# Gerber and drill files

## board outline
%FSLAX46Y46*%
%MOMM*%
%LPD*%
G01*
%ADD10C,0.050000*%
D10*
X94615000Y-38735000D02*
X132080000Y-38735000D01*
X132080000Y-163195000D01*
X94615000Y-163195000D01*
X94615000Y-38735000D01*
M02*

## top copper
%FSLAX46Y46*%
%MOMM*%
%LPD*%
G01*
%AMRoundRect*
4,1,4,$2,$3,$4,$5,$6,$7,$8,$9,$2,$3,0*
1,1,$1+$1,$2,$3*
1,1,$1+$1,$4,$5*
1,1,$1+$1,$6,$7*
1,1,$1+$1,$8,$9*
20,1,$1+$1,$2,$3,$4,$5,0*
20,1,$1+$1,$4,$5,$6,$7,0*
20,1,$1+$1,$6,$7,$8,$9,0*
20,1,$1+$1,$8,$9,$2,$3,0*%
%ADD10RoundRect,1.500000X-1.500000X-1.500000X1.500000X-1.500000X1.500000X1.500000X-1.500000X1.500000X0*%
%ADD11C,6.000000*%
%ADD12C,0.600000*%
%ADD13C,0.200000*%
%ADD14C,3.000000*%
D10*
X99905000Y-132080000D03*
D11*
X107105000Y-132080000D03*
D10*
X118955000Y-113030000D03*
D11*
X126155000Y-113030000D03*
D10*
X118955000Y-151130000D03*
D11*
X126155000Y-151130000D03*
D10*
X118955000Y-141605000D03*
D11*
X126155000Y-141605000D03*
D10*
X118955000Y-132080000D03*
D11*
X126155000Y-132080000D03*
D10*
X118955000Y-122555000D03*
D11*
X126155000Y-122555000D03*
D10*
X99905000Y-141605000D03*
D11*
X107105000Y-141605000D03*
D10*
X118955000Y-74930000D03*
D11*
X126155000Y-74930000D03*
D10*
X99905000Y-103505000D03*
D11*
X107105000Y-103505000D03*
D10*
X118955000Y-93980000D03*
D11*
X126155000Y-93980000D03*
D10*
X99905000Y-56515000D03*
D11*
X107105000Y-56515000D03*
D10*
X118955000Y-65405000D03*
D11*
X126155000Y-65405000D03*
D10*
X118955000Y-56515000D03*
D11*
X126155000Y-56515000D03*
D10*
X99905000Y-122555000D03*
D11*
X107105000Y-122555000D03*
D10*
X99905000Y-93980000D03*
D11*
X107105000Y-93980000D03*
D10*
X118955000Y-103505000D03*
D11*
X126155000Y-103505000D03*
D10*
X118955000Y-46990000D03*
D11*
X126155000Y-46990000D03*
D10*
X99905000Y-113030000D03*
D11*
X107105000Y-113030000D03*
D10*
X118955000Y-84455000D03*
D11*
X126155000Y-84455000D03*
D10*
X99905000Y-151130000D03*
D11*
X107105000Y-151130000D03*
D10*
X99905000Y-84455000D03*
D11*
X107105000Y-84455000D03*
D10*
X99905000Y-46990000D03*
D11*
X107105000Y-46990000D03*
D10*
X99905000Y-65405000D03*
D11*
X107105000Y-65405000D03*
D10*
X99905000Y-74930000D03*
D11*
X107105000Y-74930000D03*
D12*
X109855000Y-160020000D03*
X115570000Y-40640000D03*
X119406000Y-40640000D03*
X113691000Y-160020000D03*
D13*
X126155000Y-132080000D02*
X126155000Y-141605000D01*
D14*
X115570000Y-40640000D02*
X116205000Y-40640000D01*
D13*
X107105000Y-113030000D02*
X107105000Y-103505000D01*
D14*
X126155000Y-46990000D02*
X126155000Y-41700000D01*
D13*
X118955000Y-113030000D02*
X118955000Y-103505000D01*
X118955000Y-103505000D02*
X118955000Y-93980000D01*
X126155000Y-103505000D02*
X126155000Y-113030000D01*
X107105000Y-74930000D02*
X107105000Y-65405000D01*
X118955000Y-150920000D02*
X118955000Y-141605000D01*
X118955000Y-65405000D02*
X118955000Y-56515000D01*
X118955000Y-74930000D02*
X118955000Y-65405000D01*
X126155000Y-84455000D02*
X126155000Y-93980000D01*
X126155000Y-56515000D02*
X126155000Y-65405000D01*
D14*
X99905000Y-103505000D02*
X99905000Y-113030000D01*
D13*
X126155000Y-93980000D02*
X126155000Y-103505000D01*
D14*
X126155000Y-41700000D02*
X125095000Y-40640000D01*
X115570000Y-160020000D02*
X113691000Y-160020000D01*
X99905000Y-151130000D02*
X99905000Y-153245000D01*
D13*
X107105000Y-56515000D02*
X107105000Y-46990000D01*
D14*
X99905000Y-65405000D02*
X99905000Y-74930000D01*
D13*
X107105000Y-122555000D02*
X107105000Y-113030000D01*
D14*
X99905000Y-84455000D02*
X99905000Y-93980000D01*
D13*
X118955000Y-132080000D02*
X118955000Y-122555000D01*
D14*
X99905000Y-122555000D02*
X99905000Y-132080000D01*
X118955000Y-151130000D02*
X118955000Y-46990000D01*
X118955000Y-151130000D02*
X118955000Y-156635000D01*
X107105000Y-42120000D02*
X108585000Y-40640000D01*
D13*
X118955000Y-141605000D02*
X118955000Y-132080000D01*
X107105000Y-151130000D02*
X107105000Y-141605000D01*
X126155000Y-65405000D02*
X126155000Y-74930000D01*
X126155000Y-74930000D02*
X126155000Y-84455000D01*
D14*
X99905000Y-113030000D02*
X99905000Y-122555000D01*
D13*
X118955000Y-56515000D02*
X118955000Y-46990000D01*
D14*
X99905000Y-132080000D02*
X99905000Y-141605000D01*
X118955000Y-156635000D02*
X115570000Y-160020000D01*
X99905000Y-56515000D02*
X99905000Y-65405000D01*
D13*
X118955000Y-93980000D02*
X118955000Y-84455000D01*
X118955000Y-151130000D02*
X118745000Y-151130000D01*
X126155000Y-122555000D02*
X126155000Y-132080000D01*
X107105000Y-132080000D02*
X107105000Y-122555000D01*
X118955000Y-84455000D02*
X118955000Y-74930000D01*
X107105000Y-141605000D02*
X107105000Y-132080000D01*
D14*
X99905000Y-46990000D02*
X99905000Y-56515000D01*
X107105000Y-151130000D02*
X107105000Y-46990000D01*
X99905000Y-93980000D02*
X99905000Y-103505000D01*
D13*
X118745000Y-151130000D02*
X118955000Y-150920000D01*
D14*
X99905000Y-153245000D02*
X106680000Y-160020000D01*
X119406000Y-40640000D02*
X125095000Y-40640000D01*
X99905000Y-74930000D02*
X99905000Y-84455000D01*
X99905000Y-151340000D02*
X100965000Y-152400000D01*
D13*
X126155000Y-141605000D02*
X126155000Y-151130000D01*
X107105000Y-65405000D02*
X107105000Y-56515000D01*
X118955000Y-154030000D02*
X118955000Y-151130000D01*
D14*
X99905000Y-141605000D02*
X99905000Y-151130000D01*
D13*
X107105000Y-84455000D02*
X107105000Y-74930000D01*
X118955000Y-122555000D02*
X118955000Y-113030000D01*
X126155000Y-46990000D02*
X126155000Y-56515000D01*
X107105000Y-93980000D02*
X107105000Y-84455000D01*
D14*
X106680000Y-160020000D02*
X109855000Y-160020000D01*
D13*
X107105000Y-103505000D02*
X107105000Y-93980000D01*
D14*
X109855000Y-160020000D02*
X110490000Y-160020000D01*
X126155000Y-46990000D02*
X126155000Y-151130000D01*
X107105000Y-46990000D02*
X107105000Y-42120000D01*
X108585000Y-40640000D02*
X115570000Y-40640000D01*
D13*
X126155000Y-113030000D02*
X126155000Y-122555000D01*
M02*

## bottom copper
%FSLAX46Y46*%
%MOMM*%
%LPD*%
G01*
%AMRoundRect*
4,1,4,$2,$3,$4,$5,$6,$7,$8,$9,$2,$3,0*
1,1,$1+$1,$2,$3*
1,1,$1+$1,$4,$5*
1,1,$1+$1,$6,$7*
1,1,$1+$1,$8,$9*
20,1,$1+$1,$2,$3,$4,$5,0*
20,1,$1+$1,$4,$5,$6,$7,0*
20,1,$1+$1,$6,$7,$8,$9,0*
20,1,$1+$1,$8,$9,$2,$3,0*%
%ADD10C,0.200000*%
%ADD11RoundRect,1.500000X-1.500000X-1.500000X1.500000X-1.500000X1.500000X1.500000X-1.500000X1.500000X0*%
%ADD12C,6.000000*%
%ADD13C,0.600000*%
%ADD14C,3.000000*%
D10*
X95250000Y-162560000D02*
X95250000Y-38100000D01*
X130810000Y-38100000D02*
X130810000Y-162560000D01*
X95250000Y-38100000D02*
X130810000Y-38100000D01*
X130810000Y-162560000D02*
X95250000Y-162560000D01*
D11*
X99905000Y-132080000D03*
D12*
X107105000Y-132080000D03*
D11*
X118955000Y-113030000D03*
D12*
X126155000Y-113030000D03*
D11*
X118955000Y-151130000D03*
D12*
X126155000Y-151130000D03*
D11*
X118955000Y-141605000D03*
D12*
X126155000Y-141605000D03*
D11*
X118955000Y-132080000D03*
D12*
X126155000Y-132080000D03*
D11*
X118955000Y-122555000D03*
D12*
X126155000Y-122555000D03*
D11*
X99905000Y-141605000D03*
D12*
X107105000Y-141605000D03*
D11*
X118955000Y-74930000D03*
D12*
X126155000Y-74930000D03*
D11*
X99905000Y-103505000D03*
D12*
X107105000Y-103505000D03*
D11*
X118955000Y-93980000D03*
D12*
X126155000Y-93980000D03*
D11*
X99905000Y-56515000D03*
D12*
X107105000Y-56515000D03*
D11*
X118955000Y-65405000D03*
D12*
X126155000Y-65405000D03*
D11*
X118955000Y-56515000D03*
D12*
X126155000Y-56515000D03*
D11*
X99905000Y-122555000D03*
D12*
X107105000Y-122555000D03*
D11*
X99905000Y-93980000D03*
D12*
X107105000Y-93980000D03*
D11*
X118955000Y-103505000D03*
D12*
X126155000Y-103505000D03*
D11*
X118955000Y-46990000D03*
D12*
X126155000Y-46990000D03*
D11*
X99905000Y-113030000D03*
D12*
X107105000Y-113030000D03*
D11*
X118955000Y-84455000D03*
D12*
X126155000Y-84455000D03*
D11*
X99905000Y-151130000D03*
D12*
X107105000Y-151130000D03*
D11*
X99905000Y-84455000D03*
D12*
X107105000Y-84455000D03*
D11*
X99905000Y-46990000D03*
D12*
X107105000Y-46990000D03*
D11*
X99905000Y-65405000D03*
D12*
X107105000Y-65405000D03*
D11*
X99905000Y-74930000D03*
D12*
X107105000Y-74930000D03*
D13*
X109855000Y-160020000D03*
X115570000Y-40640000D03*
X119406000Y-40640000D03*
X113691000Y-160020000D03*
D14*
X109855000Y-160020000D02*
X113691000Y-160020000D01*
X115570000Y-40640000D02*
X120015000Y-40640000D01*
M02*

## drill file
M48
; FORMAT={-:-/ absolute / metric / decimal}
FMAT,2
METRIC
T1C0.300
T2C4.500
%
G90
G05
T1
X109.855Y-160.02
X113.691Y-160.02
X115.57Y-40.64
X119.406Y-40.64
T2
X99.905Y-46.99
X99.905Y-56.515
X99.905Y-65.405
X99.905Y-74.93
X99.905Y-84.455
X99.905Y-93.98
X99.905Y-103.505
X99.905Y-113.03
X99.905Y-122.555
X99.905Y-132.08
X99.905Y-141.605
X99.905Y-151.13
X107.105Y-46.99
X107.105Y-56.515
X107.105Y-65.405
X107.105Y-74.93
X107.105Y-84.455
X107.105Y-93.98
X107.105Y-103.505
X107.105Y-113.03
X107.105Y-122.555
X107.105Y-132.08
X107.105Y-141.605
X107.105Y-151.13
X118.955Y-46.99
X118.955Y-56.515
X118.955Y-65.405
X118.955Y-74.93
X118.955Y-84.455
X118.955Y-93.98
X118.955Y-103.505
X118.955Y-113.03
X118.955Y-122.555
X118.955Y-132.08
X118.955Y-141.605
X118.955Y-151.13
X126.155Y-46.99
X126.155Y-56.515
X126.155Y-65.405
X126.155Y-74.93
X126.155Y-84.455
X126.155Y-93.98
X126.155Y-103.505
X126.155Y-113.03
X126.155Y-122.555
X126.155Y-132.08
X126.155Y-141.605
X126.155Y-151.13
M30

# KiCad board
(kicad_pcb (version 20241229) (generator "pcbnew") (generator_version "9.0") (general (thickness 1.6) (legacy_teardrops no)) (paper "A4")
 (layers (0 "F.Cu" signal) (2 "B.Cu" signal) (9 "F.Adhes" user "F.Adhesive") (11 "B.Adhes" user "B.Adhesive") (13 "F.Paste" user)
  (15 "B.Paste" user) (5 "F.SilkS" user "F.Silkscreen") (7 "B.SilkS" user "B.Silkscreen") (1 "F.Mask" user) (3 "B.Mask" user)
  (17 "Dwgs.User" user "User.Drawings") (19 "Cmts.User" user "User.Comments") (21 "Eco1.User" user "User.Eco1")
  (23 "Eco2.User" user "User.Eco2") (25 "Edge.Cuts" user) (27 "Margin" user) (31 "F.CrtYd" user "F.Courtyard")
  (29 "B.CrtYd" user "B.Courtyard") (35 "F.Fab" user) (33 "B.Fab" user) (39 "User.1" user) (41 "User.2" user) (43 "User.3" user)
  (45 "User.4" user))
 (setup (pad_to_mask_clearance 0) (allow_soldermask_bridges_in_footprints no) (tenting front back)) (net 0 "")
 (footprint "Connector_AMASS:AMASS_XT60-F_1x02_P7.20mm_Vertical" (layer "F.Cu") (at 99.905 132.08)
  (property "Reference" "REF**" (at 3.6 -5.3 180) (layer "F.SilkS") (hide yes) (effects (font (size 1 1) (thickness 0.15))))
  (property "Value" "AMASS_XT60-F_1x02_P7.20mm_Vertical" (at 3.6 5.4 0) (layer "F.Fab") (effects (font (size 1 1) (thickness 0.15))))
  (pad "1" thru_hole roundrect (at 0 0) (size 6 6) (drill 4.5) (layers "*.Cu" "*.Mask") (remove_unused_layers no) (roundrect_rratio 0.25))
  (pad "2" thru_hole circle (at 7.2 0) (size 6 6) (drill 4.5) (layers "*.Cu" "*.Mask") (remove_unused_layers no)))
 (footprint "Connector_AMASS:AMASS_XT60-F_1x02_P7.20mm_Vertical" (layer "F.Cu") (at 118.955 113.03)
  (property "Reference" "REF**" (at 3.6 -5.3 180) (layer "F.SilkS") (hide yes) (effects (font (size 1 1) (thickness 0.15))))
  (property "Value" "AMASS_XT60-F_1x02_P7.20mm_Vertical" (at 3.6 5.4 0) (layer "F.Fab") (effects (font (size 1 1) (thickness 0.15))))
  (pad "1" thru_hole roundrect (at 0 0) (size 6 6) (drill 4.5) (layers "*.Cu" "*.Mask") (remove_unused_layers no) (roundrect_rratio 0.25))
  (pad "2" thru_hole circle (at 7.2 0) (size 6 6) (drill 4.5) (layers "*.Cu" "*.Mask") (remove_unused_layers no)))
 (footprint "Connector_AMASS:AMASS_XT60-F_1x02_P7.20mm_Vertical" (layer "F.Cu") (at 118.955 151.13)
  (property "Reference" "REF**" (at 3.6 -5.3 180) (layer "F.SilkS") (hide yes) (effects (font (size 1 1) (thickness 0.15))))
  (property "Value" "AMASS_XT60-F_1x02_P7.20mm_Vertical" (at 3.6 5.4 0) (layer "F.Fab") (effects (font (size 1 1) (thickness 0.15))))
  (pad "1" thru_hole roundrect (at 0 0) (size 6 6) (drill 4.5) (layers "*.Cu" "*.Mask") (remove_unused_layers no) (roundrect_rratio 0.25))
  (pad "2" thru_hole circle (at 7.2 0) (size 6 6) (drill 4.5) (layers "*.Cu" "*.Mask") (remove_unused_layers no)))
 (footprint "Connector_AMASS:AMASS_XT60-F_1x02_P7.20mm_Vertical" (layer "F.Cu") (at 118.955 141.605)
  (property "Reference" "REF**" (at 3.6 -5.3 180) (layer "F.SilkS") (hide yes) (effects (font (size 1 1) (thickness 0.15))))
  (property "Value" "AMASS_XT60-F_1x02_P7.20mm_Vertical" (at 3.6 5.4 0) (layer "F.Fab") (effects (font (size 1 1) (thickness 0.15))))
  (pad "1" thru_hole roundrect (at 0 0) (size 6 6) (drill 4.5) (layers "*.Cu" "*.Mask") (remove_unused_layers no) (roundrect_rratio 0.25))
  (pad "2" thru_hole circle (at 7.2 0) (size 6 6) (drill 4.5) (layers "*.Cu" "*.Mask") (remove_unused_layers no)))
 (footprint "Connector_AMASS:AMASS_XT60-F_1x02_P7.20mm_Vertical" (layer "F.Cu") (at 118.955 132.08)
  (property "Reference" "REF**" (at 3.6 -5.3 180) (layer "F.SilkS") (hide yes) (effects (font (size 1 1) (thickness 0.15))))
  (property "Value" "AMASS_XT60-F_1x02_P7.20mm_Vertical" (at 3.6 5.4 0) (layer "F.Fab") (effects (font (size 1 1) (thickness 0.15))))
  (pad "1" thru_hole roundrect (at 0 0) (size 6 6) (drill 4.5) (layers "*.Cu" "*.Mask") (remove_unused_layers no) (roundrect_rratio 0.25))
  (pad "2" thru_hole circle (at 7.2 0) (size 6 6) (drill 4.5) (layers "*.Cu" "*.Mask") (remove_unused_layers no)))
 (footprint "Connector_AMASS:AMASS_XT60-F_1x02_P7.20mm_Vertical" (layer "F.Cu") (at 118.955 122.555)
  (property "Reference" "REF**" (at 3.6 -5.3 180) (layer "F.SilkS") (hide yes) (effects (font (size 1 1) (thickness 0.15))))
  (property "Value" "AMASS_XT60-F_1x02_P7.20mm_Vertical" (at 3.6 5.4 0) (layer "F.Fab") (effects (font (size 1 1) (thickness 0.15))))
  (pad "1" thru_hole roundrect (at 0 0) (size 6 6) (drill 4.5) (layers "*.Cu" "*.Mask") (remove_unused_layers no) (roundrect_rratio 0.25))
  (pad "2" thru_hole circle (at 7.2 0) (size 6 6) (drill 4.5) (layers "*.Cu" "*.Mask") (remove_unused_layers no)))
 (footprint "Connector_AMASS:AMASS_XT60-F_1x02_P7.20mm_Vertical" (layer "F.Cu") (at 99.905 141.605)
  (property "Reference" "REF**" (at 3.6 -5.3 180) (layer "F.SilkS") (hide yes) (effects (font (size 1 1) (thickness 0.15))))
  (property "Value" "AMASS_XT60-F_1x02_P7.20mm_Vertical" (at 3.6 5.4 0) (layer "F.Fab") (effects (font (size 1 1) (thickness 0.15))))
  (pad "1" thru_hole roundrect (at 0 0) (size 6 6) (drill 4.5) (layers "*.Cu" "*.Mask") (remove_unused_layers no) (roundrect_rratio 0.25))
  (pad "2" thru_hole circle (at 7.2 0) (size 6 6) (drill 4.5) (layers "*.Cu" "*.Mask") (remove_unused_layers no)))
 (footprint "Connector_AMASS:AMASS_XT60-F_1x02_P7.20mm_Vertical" (layer "F.Cu") (at 118.955 74.93)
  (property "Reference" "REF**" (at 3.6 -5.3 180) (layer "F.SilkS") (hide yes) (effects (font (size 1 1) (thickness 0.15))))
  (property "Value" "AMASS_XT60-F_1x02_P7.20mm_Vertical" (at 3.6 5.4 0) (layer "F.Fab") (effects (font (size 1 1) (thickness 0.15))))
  (pad "1" thru_hole roundrect (at 0 0) (size 6 6) (drill 4.5) (layers "*.Cu" "*.Mask") (remove_unused_layers no) (roundrect_rratio 0.25))
  (pad "2" thru_hole circle (at 7.2 0) (size 6 6) (drill 4.5) (layers "*.Cu" "*.Mask") (remove_unused_layers no)))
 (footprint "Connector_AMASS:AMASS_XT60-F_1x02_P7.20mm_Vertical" (layer "F.Cu") (at 99.905 103.505)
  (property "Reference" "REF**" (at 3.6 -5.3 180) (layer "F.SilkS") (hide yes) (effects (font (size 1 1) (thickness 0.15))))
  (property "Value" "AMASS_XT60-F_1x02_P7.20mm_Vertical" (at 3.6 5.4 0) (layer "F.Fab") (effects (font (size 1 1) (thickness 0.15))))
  (pad "1" thru_hole roundrect (at 0 0) (size 6 6) (drill 4.5) (layers "*.Cu" "*.Mask") (remove_unused_layers no) (roundrect_rratio 0.25))
  (pad "2" thru_hole circle (at 7.2 0) (size 6 6) (drill 4.5) (layers "*.Cu" "*.Mask") (remove_unused_layers no)))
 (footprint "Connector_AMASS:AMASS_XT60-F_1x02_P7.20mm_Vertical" (layer "F.Cu") (at 118.955 93.98)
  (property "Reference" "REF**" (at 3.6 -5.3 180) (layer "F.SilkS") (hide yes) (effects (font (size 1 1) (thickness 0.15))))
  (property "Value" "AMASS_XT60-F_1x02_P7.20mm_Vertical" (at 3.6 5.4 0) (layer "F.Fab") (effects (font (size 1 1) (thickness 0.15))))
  (pad "1" thru_hole roundrect (at 0 0) (size 6 6) (drill 4.5) (layers "*.Cu" "*.Mask") (remove_unused_layers no) (roundrect_rratio 0.25))
  (pad "2" thru_hole circle (at 7.2 0) (size 6 6) (drill 4.5) (layers "*.Cu" "*.Mask") (remove_unused_layers no)))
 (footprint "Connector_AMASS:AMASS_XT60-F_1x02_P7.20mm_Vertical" (layer "F.Cu") (at 99.905 56.515)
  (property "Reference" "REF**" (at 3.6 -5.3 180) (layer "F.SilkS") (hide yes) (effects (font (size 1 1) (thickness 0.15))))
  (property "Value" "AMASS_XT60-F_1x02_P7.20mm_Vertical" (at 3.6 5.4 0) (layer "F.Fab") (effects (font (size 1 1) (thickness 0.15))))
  (pad "1" thru_hole roundrect (at 0 0) (size 6 6) (drill 4.5) (layers "*.Cu" "*.Mask") (remove_unused_layers no) (roundrect_rratio 0.25))
  (pad "2" thru_hole circle (at 7.2 0) (size 6 6) (drill 4.5) (layers "*.Cu" "*.Mask") (remove_unused_layers no)))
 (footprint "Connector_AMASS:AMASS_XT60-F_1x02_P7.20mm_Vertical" (layer "F.Cu") (at 118.955 65.405)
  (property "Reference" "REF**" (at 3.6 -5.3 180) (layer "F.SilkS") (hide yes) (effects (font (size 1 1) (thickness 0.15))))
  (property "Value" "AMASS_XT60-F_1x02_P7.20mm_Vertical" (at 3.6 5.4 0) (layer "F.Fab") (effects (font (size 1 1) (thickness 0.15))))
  (pad "1" thru_hole roundrect (at 0 0) (size 6 6) (drill 4.5) (layers "*.Cu" "*.Mask") (remove_unused_layers no) (roundrect_rratio 0.25))
  (pad "2" thru_hole circle (at 7.2 0) (size 6 6) (drill 4.5) (layers "*.Cu" "*.Mask") (remove_unused_layers no)))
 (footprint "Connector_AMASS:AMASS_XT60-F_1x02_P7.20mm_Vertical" (layer "F.Cu") (at 118.955 56.515)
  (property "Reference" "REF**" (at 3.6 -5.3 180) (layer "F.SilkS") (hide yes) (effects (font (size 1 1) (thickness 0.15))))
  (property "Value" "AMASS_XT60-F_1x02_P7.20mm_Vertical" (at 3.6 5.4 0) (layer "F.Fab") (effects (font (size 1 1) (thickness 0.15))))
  (pad "1" thru_hole roundrect (at 0 0) (size 6 6) (drill 4.5) (layers "*.Cu" "*.Mask") (remove_unused_layers no) (roundrect_rratio 0.25))
  (pad "2" thru_hole circle (at 7.2 0) (size 6 6) (drill 4.5) (layers "*.Cu" "*.Mask") (remove_unused_layers no)))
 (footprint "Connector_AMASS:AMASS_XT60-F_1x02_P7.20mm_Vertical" (layer "F.Cu") (at 99.905 122.555)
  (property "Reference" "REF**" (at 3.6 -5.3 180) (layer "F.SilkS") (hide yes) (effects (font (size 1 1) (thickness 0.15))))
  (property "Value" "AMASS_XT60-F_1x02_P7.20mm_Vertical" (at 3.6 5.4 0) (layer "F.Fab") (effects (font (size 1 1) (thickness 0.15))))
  (pad "1" thru_hole roundrect (at 0 0) (size 6 6) (drill 4.5) (layers "*.Cu" "*.Mask") (remove_unused_layers no) (roundrect_rratio 0.25))
  (pad "2" thru_hole circle (at 7.2 0) (size 6 6) (drill 4.5) (layers "*.Cu" "*.Mask") (remove_unused_layers no)))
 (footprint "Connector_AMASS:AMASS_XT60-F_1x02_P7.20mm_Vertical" (layer "F.Cu") (at 99.905 93.98)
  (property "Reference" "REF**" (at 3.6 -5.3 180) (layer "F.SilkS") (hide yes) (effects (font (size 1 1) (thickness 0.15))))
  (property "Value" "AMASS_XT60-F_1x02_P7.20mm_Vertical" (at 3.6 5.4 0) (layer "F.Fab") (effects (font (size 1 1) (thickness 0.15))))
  (pad "1" thru_hole roundrect (at 0 0) (size 6 6) (drill 4.5) (layers "*.Cu" "*.Mask") (remove_unused_layers no) (roundrect_rratio 0.25))
  (pad "2" thru_hole circle (at 7.2 0) (size 6 6) (drill 4.5) (layers "*.Cu" "*.Mask") (remove_unused_layers no)))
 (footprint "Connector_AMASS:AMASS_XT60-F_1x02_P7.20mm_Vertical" (layer "F.Cu") (at 118.955 103.505)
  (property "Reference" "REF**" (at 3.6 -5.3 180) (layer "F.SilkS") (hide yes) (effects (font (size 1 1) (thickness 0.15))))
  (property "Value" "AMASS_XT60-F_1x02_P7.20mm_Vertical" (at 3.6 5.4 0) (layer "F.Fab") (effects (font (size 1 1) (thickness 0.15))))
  (pad "1" thru_hole roundrect (at 0 0) (size 6 6) (drill 4.5) (layers "*.Cu" "*.Mask") (remove_unused_layers no) (roundrect_rratio 0.25))
  (pad "2" thru_hole circle (at 7.2 0) (size 6 6) (drill 4.5) (layers "*.Cu" "*.Mask") (remove_unused_layers no)))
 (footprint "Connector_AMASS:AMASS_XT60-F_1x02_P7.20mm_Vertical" (layer "F.Cu") (at 118.955 46.99)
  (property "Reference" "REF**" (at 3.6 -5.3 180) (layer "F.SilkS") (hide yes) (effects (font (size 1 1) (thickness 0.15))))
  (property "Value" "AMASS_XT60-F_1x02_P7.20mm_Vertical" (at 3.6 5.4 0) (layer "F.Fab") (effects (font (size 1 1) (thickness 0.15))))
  (pad "1" thru_hole roundrect (at 0 0) (size 6 6) (drill 4.5) (layers "*.Cu" "*.Mask") (remove_unused_layers no) (roundrect_rratio 0.25))
  (pad "2" thru_hole circle (at 7.2 0) (size 6 6) (drill 4.5) (layers "*.Cu" "*.Mask") (remove_unused_layers no)))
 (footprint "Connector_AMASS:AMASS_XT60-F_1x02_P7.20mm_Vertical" (layer "F.Cu") (at 99.905 113.03)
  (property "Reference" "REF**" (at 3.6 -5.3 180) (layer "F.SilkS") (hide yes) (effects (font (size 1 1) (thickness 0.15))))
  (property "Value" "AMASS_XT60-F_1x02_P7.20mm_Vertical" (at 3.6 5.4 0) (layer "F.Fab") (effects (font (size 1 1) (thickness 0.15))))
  (pad "1" thru_hole roundrect (at 0 0) (size 6 6) (drill 4.5) (layers "*.Cu" "*.Mask") (remove_unused_layers no) (roundrect_rratio 0.25))
  (pad "2" thru_hole circle (at 7.2 0) (size 6 6) (drill 4.5) (layers "*.Cu" "*.Mask") (remove_unused_layers no)))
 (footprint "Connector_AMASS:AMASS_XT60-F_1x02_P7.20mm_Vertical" (layer "F.Cu") (at 118.955 84.455)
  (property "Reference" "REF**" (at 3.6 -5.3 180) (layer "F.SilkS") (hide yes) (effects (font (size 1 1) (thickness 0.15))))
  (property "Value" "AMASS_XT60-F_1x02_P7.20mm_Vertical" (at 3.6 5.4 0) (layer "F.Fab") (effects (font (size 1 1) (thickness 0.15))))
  (pad "1" thru_hole roundrect (at 0 0) (size 6 6) (drill 4.5) (layers "*.Cu" "*.Mask") (remove_unused_layers no) (roundrect_rratio 0.25))
  (pad "2" thru_hole circle (at 7.2 0) (size 6 6) (drill 4.5) (layers "*.Cu" "*.Mask") (remove_unused_layers no)))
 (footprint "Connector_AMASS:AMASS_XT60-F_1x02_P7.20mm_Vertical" (layer "F.Cu") (at 99.905 151.13)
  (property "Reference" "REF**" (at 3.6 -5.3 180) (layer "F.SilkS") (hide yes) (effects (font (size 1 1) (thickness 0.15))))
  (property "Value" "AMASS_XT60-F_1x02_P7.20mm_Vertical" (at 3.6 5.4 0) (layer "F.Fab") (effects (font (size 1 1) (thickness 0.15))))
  (pad "1" thru_hole roundrect (at 0 0) (size 6 6) (drill 4.5) (layers "*.Cu" "*.Mask") (remove_unused_layers no) (roundrect_rratio 0.25))
  (pad "2" thru_hole circle (at 7.2 0) (size 6 6) (drill 4.5) (layers "*.Cu" "*.Mask") (remove_unused_layers no)))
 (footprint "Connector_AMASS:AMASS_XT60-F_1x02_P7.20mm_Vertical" (layer "F.Cu") (at 99.905 84.455)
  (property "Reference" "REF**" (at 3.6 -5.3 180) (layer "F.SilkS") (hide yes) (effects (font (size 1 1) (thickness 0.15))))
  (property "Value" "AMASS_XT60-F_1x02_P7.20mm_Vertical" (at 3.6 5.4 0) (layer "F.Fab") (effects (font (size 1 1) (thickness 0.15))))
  (pad "1" thru_hole roundrect (at 0 0) (size 6 6) (drill 4.5) (layers "*.Cu" "*.Mask") (remove_unused_layers no) (roundrect_rratio 0.25))
  (pad "2" thru_hole circle (at 7.2 0) (size 6 6) (drill 4.5) (layers "*.Cu" "*.Mask") (remove_unused_layers no)))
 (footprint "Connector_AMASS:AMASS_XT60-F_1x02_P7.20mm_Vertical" (layer "F.Cu") (at 99.905 46.99)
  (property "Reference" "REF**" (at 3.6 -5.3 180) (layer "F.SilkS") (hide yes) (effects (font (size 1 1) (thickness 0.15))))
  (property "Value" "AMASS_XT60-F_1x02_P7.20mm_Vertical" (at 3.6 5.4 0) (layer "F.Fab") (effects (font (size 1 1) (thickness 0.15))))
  (pad "1" thru_hole roundrect (at 0 0) (size 6 6) (drill 4.5) (layers "*.Cu" "*.Mask") (remove_unused_layers no) (roundrect_rratio 0.25))
  (pad "2" thru_hole circle (at 7.2 0) (size 6 6) (drill 4.5) (layers "*.Cu" "*.Mask") (remove_unused_layers no)))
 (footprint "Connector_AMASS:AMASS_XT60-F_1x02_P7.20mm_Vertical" (layer "F.Cu") (at 99.905 65.405)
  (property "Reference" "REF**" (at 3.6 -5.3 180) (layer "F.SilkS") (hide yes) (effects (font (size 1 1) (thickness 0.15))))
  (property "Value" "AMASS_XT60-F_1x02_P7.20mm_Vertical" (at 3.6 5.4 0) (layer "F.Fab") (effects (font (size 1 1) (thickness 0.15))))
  (pad "1" thru_hole roundrect (at 0 0) (size 6 6) (drill 4.5) (layers "*.Cu" "*.Mask") (remove_unused_layers no) (roundrect_rratio 0.25))
  (pad "2" thru_hole circle (at 7.2 0) (size 6 6) (drill 4.5) (layers "*.Cu" "*.Mask") (remove_unused_layers no)))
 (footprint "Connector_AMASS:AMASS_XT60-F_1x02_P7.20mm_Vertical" (layer "F.Cu") (at 99.905 74.93)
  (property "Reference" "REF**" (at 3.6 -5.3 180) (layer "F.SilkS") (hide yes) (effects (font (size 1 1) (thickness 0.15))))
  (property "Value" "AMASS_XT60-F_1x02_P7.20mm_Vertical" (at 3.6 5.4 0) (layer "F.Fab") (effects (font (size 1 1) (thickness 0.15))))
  (pad "1" thru_hole roundrect (at 0 0) (size 6 6) (drill 4.5) (layers "*.Cu" "*.Mask") (remove_unused_layers no) (roundrect_rratio 0.25))
  (pad "2" thru_hole circle (at 7.2 0) (size 6 6) (drill 4.5) (layers "*.Cu" "*.Mask") (remove_unused_layers no)))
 (gr_line (start 95.25 162.56) (end 95.25 38.1) (stroke (width 0.2) (type default)) (layer "B.Cu"))
 (gr_line (start 130.81 38.1) (end 130.81 162.56) (stroke (width 0.2) (type default)) (layer "B.Cu"))
 (gr_line (start 95.25 38.1) (end 130.81 38.1) (stroke (width 0.2) (type default)) (layer "B.Cu"))
 (gr_line (start 130.81 162.56) (end 95.25 162.56) (stroke (width 0.2) (type default)) (layer "B.Cu"))
 (gr_rect (start 94.615 38.735) (end 132.08 163.195) (stroke (width 0.05) (type default)) (fill no) (layer "Edge.Cuts"))
 (segment (start 126.155 132.08) (end 126.155 141.605) (width 0.2) (layer "F.Cu") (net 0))
 (segment (start 115.57 40.64) (end 116.205 40.64) (width 3) (layer "F.Cu") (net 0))
 (segment (start 107.105 113.03) (end 107.105 103.505) (width 0.2) (layer "F.Cu") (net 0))
 (segment (start 126.155 46.99) (end 126.155 41.7) (width 3) (layer "F.Cu") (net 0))
 (segment (start 118.955 113.03) (end 118.955 103.505) (width 0.2) (layer "F.Cu") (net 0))
 (segment (start 118.955 103.505) (end 118.955 93.98) (width 0.2) (layer "F.Cu") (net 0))
 (segment (start 126.155 103.505) (end 126.155 113.03) (width 0.2) (layer "F.Cu") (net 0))
 (segment (start 107.105 74.93) (end 107.105 65.405) (width 0.2) (layer "F.Cu") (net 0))
 (segment (start 118.955 150.92) (end 118.955 141.605) (width 0.2) (layer "F.Cu") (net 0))
 (segment (start 118.955 65.405) (end 118.955 56.515) (width 0.2) (layer "F.Cu") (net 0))
 (segment (start 118.955 74.93) (end 118.955 65.405) (width 0.2) (layer "F.Cu") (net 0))
 (segment (start 126.155 84.455) (end 126.155 93.98) (width 0.2) (layer "F.Cu") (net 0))
 (segment (start 126.155 56.515) (end 126.155 65.405) (width 0.2) (layer "F.Cu") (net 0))
 (segment (start 99.905 103.505) (end 99.905 113.03) (width 3) (layer "F.Cu") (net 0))
 (segment (start 126.155 93.98) (end 126.155 103.505) (width 0.2) (layer "F.Cu") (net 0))
 (segment (start 126.155 41.7) (end 125.095 40.64) (width 3) (layer "F.Cu") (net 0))
 (segment (start 115.57 160.02) (end 113.691 160.02) (width 3) (layer "F.Cu") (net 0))
 (segment (start 99.905 151.13) (end 99.905 153.245) (width 3) (layer "F.Cu") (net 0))
 (segment (start 107.105 56.515) (end 107.105 46.99) (width 0.2) (layer "F.Cu") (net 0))
 (segment (start 99.905 65.405) (end 99.905 74.93) (width 3) (layer "F.Cu") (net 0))
 (segment (start 107.105 122.555) (end 107.105 113.03) (width 0.2) (layer "F.Cu") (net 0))
 (segment (start 99.905 84.455) (end 99.905 93.98) (width 3) (layer "F.Cu") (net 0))
 (segment (start 118.955 132.08) (end 118.955 122.555) (width 0.2) (layer "F.Cu") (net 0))
 (segment (start 99.905 122.555) (end 99.905 132.08) (width 3) (layer "F.Cu") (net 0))
 (segment (start 118.955 151.13) (end 118.955 46.99) (width 3) (layer "F.Cu") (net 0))
 (segment (start 118.955 151.13) (end 118.955 156.635) (width 3) (layer "F.Cu") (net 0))
 (segment (start 107.105 42.12) (end 108.585 40.64) (width 3) (layer "F.Cu") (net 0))
 (segment (start 118.955 141.605) (end 118.955 132.08) (width 0.2) (layer "F.Cu") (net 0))
 (segment (start 107.105 151.13) (end 107.105 141.605) (width 0.2) (layer "F.Cu") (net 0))
 (segment (start 126.155 65.405) (end 126.155 74.93) (width 0.2) (layer "F.Cu") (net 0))
 (segment (start 126.155 74.93) (end 126.155 84.455) (width 0.2) (layer "F.Cu") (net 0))
 (segment (start 99.905 113.03) (end 99.905 122.555) (width 3) (layer "F.Cu") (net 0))
 (segment (start 118.955 56.515) (end 118.955 46.99) (width 0.2) (layer "F.Cu") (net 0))
 (segment (start 99.905 132.08) (end 99.905 141.605) (width 3) (layer "F.Cu") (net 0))
 (segment (start 118.955 156.635) (end 115.57 160.02) (width 3) (layer "F.Cu") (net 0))
 (segment (start 99.905 56.515) (end 99.905 65.405) (width 3) (layer "F.Cu") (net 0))
 (segment (start 118.955 93.98) (end 118.955 84.455) (width 0.2) (layer "F.Cu") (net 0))
 (segment (start 118.955 151.13) (end 118.745 151.13) (width 0.2) (layer "F.Cu") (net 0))
 (segment (start 126.155 122.555) (end 126.155 132.08) (width 0.2) (layer "F.Cu") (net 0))
 (segment (start 107.105 132.08) (end 107.105 122.555) (width 0.2) (layer "F.Cu") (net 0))
 (segment (start 118.955 84.455) (end 118.955 74.93) (width 0.2) (layer "F.Cu") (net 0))
 (segment (start 107.105 141.605) (end 107.105 132.08) (width 0.2) (layer "F.Cu") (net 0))
 (segment (start 99.905 46.99) (end 99.905 56.515) (width 3) (layer "F.Cu") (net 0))
 (segment (start 107.105 151.13) (end 107.105 46.99) (width 3) (layer "F.Cu") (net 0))
 (segment (start 99.905 93.98) (end 99.905 103.505) (width 3) (layer "F.Cu") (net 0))
 (segment (start 118.745 151.13) (end 118.955 150.92) (width 0.2) (layer "F.Cu") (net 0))
 (segment (start 99.905 153.245) (end 106.68 160.02) (width 3) (layer "F.Cu") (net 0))
 (segment (start 119.406 40.64) (end 125.095 40.64) (width 3) (layer "F.Cu") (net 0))
 (segment (start 99.905 74.93) (end 99.905 84.455) (width 3) (layer "F.Cu") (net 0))
 (segment (start 99.905 151.34) (end 100.965 152.4) (width 3) (layer "F.Cu") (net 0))
 (segment (start 126.155 141.605) (end 126.155 151.13) (width 0.2) (layer "F.Cu") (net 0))
 (segment (start 107.105 65.405) (end 107.105 56.515) (width 0.2) (layer "F.Cu") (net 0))
 (segment (start 118.955 154.03) (end 118.955 151.13) (width 0.2) (layer "F.Cu") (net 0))
 (segment (start 99.905 141.605) (end 99.905 151.13) (width 3) (layer "F.Cu") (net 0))
 (segment (start 107.105 84.455) (end 107.105 74.93) (width 0.2) (layer "F.Cu") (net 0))
 (segment (start 118.955 122.555) (end 118.955 113.03) (width 0.2) (layer "F.Cu") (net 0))
 (segment (start 126.155 46.99) (end 126.155 56.515) (width 0.2) (layer "F.Cu") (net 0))
 (segment (start 107.105 93.98) (end 107.105 84.455) (width 0.2) (layer "F.Cu") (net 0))
 (segment (start 106.68 160.02) (end 109.855 160.02) (width 3) (layer "F.Cu") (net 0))
 (segment (start 107.105 103.505) (end 107.105 93.98) (width 0.2) (layer "F.Cu") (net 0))
 (segment (start 109.855 160.02) (end 110.49 160.02) (width 3) (layer "F.Cu") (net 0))
 (segment (start 126.155 46.99) (end 126.155 151.13) (width 3) (layer "F.Cu") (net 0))
 (segment (start 107.105 46.99) (end 107.105 42.12) (width 3) (layer "F.Cu") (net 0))
 (segment (start 108.585 40.64) (end 115.57 40.64) (width 3) (layer "F.Cu") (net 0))
 (segment (start 126.155 113.03) (end 126.155 122.555) (width 0.2) (layer "F.Cu") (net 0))
 (via (at 109.855 160.02) (size 0.6) (drill 0.3) (layers "F.Cu" "B.Cu") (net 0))
 (via (at 115.57 40.64) (size 0.6) (drill 0.3) (layers "F.Cu" "B.Cu") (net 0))
 (via (at 119.406 40.64) (size 0.6) (drill 0.3) (layers "F.Cu" "B.Cu") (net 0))
 (via (at 113.691 160.02) (size 0.6) (drill 0.3) (layers "F.Cu" "B.Cu") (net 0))
 (segment (start 109.855 160.02) (end 113.691 160.02) (width 3) (layer "B.Cu") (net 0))
 (segment (start 115.57 40.64) (end 120.015 40.64) (width 3) (layer "B.Cu") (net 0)))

